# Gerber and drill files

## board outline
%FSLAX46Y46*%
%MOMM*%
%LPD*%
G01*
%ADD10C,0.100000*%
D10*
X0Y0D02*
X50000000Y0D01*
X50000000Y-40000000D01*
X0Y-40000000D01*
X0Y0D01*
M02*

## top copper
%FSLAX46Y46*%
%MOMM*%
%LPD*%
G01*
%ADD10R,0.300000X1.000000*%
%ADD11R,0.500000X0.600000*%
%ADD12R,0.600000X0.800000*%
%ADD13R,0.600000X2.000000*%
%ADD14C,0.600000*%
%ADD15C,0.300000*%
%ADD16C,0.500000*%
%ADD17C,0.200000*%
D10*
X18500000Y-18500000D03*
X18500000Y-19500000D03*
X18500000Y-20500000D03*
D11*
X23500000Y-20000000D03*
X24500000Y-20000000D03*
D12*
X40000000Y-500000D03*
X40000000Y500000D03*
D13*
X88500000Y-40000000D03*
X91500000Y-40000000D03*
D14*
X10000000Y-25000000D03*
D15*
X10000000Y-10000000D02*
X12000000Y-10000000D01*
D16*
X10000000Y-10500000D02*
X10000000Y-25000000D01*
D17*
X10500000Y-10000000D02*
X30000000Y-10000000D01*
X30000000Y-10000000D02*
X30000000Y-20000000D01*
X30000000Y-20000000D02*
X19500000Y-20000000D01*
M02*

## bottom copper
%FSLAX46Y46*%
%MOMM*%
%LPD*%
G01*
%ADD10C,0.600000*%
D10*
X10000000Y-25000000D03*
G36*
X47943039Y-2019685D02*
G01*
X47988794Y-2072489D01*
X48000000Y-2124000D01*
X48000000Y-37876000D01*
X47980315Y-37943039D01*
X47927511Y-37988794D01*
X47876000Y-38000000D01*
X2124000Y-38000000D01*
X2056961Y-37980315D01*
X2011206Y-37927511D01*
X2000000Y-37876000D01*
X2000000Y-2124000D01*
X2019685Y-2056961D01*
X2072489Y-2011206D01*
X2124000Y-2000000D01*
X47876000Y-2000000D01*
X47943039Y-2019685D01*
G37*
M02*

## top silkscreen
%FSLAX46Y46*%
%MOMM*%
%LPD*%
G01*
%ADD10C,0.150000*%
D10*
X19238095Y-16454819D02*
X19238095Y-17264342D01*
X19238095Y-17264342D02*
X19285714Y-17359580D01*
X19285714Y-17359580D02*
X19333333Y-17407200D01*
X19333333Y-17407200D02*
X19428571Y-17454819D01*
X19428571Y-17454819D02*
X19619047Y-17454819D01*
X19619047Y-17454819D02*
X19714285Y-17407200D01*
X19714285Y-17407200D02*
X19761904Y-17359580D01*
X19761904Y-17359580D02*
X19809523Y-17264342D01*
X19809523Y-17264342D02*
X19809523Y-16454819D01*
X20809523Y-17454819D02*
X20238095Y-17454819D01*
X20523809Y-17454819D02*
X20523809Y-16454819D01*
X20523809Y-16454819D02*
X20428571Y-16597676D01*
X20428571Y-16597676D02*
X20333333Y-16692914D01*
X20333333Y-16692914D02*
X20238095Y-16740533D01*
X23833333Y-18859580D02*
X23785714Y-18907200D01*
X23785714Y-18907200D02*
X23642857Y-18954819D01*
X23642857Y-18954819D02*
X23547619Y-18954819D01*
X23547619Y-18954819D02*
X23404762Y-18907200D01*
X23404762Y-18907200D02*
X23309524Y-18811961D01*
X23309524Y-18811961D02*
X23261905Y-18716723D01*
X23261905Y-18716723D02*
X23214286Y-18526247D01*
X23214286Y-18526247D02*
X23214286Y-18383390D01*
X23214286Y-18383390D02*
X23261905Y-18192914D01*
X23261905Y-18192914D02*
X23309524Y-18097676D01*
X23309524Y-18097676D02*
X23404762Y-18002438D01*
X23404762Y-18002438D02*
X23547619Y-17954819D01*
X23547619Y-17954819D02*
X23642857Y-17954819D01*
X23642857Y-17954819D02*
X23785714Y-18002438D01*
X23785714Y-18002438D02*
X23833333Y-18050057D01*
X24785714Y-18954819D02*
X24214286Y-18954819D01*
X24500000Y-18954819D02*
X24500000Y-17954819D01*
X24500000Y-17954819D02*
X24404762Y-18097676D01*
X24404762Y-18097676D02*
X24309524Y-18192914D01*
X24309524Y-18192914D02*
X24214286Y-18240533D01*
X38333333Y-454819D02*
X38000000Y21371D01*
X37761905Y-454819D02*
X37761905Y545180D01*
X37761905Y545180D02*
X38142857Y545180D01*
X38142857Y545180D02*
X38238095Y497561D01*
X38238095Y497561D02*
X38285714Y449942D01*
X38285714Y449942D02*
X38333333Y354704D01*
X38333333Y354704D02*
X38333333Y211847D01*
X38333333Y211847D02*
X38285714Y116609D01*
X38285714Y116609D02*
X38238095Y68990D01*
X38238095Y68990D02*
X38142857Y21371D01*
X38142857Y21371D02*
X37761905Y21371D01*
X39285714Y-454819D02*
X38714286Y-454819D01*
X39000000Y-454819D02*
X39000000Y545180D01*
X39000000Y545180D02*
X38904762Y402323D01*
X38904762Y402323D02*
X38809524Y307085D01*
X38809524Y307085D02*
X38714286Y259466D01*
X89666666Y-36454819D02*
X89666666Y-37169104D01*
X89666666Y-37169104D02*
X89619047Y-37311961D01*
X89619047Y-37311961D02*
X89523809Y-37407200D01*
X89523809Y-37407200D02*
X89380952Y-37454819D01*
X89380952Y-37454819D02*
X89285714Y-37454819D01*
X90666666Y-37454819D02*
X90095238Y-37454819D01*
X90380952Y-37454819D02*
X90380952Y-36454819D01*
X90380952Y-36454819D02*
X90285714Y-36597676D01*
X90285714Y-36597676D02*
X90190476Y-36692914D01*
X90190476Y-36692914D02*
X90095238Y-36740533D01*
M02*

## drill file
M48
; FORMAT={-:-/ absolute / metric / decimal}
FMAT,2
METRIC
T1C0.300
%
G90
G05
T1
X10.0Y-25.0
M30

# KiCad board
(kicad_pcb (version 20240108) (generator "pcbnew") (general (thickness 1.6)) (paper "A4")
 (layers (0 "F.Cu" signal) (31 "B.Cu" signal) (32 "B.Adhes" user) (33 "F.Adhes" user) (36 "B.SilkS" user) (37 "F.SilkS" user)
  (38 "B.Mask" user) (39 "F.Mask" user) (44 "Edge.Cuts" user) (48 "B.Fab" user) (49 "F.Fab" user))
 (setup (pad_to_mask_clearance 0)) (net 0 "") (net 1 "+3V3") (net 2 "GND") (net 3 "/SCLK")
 (gr_rect (start 0 0) (end 50 40) (layer "Edge.Cuts") (width 0.1))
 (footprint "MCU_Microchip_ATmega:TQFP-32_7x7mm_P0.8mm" (layer "F.Cu") (at 10 10 0)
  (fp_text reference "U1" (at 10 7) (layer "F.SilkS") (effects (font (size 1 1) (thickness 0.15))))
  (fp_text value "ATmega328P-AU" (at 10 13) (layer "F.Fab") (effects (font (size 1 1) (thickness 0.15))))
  (pad "1" smd rect (at 8.5 8.5) (size 0.3 1) (layers "F.Cu" "F.Paste" "F.Mask") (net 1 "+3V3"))
  (pad "2" smd rect (at 8.5 9.5) (size 0.3 1) (layers "F.Cu" "F.Paste" "F.Mask") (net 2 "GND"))
  (pad "3" smd rect (at 8.5 10.5) (size 0.3 1) (layers "F.Cu" "F.Paste" "F.Mask") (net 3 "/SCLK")))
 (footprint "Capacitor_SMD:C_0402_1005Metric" (layer "F.Cu") (at 12 10 0)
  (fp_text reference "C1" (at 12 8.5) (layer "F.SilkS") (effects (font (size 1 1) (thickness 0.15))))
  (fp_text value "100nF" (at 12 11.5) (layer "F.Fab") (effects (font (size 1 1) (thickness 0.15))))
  (pad "1" smd rect (at 11.5 10) (size 0.5 0.6) (layers "F.Cu" "F.Paste" "F.Mask") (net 1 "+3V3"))
  (pad "2" smd rect (at 12.5 10) (size 0.5 0.6) (layers "F.Cu" "F.Paste" "F.Mask") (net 2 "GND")))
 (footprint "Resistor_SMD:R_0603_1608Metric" (layer "F.Cu") (at 20 20 90)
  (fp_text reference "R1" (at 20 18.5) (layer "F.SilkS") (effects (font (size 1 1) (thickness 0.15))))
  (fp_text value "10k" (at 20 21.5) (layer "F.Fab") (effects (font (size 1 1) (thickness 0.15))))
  (pad "1" smd rect (at 19.5 20) (size 0.6 0.8) (layers "F.Cu" "F.Paste" "F.Mask") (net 3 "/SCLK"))
  (pad "2" smd rect (at 20.5 20) (size 0.6 0.8) (layers "F.Cu" "F.Paste" "F.Mask") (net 2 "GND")))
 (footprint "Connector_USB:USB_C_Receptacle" (layer "F.Cu") (at 45 20 0)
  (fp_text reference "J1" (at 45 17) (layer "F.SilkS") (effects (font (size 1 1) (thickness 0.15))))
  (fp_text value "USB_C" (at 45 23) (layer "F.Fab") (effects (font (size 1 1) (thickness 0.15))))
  (pad "1" smd rect (at 43.5 20) (size 0.6 2) (layers "F.Cu" "F.Paste" "F.Mask") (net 1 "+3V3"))
  (pad "2" smd rect (at 46.5 20) (size 0.6 2) (layers "F.Cu" "F.Paste" "F.Mask") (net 2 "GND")))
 (segment (start 10 10) (end 12 10) (width 0.3) (layer "F.Cu") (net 1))
 (segment (start 10 10.5) (end 10 25) (width 0.5) (layer "F.Cu") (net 2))
 (segment (start 10.5 10) (end 30 10) (width 0.2) (layer "F.Cu") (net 3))
 (segment (start 30 10) (end 30 20) (width 0.2) (layer "F.Cu") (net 3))
 (segment (start 30 20) (end 19.5 20) (width 0.2) (layer "F.Cu") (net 3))
 (via (at 10 25) (size 0.6) (drill 0.3) (layers "F.Cu" "B.Cu") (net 2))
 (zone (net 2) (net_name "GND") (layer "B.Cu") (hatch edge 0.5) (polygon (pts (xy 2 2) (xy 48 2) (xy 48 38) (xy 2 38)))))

